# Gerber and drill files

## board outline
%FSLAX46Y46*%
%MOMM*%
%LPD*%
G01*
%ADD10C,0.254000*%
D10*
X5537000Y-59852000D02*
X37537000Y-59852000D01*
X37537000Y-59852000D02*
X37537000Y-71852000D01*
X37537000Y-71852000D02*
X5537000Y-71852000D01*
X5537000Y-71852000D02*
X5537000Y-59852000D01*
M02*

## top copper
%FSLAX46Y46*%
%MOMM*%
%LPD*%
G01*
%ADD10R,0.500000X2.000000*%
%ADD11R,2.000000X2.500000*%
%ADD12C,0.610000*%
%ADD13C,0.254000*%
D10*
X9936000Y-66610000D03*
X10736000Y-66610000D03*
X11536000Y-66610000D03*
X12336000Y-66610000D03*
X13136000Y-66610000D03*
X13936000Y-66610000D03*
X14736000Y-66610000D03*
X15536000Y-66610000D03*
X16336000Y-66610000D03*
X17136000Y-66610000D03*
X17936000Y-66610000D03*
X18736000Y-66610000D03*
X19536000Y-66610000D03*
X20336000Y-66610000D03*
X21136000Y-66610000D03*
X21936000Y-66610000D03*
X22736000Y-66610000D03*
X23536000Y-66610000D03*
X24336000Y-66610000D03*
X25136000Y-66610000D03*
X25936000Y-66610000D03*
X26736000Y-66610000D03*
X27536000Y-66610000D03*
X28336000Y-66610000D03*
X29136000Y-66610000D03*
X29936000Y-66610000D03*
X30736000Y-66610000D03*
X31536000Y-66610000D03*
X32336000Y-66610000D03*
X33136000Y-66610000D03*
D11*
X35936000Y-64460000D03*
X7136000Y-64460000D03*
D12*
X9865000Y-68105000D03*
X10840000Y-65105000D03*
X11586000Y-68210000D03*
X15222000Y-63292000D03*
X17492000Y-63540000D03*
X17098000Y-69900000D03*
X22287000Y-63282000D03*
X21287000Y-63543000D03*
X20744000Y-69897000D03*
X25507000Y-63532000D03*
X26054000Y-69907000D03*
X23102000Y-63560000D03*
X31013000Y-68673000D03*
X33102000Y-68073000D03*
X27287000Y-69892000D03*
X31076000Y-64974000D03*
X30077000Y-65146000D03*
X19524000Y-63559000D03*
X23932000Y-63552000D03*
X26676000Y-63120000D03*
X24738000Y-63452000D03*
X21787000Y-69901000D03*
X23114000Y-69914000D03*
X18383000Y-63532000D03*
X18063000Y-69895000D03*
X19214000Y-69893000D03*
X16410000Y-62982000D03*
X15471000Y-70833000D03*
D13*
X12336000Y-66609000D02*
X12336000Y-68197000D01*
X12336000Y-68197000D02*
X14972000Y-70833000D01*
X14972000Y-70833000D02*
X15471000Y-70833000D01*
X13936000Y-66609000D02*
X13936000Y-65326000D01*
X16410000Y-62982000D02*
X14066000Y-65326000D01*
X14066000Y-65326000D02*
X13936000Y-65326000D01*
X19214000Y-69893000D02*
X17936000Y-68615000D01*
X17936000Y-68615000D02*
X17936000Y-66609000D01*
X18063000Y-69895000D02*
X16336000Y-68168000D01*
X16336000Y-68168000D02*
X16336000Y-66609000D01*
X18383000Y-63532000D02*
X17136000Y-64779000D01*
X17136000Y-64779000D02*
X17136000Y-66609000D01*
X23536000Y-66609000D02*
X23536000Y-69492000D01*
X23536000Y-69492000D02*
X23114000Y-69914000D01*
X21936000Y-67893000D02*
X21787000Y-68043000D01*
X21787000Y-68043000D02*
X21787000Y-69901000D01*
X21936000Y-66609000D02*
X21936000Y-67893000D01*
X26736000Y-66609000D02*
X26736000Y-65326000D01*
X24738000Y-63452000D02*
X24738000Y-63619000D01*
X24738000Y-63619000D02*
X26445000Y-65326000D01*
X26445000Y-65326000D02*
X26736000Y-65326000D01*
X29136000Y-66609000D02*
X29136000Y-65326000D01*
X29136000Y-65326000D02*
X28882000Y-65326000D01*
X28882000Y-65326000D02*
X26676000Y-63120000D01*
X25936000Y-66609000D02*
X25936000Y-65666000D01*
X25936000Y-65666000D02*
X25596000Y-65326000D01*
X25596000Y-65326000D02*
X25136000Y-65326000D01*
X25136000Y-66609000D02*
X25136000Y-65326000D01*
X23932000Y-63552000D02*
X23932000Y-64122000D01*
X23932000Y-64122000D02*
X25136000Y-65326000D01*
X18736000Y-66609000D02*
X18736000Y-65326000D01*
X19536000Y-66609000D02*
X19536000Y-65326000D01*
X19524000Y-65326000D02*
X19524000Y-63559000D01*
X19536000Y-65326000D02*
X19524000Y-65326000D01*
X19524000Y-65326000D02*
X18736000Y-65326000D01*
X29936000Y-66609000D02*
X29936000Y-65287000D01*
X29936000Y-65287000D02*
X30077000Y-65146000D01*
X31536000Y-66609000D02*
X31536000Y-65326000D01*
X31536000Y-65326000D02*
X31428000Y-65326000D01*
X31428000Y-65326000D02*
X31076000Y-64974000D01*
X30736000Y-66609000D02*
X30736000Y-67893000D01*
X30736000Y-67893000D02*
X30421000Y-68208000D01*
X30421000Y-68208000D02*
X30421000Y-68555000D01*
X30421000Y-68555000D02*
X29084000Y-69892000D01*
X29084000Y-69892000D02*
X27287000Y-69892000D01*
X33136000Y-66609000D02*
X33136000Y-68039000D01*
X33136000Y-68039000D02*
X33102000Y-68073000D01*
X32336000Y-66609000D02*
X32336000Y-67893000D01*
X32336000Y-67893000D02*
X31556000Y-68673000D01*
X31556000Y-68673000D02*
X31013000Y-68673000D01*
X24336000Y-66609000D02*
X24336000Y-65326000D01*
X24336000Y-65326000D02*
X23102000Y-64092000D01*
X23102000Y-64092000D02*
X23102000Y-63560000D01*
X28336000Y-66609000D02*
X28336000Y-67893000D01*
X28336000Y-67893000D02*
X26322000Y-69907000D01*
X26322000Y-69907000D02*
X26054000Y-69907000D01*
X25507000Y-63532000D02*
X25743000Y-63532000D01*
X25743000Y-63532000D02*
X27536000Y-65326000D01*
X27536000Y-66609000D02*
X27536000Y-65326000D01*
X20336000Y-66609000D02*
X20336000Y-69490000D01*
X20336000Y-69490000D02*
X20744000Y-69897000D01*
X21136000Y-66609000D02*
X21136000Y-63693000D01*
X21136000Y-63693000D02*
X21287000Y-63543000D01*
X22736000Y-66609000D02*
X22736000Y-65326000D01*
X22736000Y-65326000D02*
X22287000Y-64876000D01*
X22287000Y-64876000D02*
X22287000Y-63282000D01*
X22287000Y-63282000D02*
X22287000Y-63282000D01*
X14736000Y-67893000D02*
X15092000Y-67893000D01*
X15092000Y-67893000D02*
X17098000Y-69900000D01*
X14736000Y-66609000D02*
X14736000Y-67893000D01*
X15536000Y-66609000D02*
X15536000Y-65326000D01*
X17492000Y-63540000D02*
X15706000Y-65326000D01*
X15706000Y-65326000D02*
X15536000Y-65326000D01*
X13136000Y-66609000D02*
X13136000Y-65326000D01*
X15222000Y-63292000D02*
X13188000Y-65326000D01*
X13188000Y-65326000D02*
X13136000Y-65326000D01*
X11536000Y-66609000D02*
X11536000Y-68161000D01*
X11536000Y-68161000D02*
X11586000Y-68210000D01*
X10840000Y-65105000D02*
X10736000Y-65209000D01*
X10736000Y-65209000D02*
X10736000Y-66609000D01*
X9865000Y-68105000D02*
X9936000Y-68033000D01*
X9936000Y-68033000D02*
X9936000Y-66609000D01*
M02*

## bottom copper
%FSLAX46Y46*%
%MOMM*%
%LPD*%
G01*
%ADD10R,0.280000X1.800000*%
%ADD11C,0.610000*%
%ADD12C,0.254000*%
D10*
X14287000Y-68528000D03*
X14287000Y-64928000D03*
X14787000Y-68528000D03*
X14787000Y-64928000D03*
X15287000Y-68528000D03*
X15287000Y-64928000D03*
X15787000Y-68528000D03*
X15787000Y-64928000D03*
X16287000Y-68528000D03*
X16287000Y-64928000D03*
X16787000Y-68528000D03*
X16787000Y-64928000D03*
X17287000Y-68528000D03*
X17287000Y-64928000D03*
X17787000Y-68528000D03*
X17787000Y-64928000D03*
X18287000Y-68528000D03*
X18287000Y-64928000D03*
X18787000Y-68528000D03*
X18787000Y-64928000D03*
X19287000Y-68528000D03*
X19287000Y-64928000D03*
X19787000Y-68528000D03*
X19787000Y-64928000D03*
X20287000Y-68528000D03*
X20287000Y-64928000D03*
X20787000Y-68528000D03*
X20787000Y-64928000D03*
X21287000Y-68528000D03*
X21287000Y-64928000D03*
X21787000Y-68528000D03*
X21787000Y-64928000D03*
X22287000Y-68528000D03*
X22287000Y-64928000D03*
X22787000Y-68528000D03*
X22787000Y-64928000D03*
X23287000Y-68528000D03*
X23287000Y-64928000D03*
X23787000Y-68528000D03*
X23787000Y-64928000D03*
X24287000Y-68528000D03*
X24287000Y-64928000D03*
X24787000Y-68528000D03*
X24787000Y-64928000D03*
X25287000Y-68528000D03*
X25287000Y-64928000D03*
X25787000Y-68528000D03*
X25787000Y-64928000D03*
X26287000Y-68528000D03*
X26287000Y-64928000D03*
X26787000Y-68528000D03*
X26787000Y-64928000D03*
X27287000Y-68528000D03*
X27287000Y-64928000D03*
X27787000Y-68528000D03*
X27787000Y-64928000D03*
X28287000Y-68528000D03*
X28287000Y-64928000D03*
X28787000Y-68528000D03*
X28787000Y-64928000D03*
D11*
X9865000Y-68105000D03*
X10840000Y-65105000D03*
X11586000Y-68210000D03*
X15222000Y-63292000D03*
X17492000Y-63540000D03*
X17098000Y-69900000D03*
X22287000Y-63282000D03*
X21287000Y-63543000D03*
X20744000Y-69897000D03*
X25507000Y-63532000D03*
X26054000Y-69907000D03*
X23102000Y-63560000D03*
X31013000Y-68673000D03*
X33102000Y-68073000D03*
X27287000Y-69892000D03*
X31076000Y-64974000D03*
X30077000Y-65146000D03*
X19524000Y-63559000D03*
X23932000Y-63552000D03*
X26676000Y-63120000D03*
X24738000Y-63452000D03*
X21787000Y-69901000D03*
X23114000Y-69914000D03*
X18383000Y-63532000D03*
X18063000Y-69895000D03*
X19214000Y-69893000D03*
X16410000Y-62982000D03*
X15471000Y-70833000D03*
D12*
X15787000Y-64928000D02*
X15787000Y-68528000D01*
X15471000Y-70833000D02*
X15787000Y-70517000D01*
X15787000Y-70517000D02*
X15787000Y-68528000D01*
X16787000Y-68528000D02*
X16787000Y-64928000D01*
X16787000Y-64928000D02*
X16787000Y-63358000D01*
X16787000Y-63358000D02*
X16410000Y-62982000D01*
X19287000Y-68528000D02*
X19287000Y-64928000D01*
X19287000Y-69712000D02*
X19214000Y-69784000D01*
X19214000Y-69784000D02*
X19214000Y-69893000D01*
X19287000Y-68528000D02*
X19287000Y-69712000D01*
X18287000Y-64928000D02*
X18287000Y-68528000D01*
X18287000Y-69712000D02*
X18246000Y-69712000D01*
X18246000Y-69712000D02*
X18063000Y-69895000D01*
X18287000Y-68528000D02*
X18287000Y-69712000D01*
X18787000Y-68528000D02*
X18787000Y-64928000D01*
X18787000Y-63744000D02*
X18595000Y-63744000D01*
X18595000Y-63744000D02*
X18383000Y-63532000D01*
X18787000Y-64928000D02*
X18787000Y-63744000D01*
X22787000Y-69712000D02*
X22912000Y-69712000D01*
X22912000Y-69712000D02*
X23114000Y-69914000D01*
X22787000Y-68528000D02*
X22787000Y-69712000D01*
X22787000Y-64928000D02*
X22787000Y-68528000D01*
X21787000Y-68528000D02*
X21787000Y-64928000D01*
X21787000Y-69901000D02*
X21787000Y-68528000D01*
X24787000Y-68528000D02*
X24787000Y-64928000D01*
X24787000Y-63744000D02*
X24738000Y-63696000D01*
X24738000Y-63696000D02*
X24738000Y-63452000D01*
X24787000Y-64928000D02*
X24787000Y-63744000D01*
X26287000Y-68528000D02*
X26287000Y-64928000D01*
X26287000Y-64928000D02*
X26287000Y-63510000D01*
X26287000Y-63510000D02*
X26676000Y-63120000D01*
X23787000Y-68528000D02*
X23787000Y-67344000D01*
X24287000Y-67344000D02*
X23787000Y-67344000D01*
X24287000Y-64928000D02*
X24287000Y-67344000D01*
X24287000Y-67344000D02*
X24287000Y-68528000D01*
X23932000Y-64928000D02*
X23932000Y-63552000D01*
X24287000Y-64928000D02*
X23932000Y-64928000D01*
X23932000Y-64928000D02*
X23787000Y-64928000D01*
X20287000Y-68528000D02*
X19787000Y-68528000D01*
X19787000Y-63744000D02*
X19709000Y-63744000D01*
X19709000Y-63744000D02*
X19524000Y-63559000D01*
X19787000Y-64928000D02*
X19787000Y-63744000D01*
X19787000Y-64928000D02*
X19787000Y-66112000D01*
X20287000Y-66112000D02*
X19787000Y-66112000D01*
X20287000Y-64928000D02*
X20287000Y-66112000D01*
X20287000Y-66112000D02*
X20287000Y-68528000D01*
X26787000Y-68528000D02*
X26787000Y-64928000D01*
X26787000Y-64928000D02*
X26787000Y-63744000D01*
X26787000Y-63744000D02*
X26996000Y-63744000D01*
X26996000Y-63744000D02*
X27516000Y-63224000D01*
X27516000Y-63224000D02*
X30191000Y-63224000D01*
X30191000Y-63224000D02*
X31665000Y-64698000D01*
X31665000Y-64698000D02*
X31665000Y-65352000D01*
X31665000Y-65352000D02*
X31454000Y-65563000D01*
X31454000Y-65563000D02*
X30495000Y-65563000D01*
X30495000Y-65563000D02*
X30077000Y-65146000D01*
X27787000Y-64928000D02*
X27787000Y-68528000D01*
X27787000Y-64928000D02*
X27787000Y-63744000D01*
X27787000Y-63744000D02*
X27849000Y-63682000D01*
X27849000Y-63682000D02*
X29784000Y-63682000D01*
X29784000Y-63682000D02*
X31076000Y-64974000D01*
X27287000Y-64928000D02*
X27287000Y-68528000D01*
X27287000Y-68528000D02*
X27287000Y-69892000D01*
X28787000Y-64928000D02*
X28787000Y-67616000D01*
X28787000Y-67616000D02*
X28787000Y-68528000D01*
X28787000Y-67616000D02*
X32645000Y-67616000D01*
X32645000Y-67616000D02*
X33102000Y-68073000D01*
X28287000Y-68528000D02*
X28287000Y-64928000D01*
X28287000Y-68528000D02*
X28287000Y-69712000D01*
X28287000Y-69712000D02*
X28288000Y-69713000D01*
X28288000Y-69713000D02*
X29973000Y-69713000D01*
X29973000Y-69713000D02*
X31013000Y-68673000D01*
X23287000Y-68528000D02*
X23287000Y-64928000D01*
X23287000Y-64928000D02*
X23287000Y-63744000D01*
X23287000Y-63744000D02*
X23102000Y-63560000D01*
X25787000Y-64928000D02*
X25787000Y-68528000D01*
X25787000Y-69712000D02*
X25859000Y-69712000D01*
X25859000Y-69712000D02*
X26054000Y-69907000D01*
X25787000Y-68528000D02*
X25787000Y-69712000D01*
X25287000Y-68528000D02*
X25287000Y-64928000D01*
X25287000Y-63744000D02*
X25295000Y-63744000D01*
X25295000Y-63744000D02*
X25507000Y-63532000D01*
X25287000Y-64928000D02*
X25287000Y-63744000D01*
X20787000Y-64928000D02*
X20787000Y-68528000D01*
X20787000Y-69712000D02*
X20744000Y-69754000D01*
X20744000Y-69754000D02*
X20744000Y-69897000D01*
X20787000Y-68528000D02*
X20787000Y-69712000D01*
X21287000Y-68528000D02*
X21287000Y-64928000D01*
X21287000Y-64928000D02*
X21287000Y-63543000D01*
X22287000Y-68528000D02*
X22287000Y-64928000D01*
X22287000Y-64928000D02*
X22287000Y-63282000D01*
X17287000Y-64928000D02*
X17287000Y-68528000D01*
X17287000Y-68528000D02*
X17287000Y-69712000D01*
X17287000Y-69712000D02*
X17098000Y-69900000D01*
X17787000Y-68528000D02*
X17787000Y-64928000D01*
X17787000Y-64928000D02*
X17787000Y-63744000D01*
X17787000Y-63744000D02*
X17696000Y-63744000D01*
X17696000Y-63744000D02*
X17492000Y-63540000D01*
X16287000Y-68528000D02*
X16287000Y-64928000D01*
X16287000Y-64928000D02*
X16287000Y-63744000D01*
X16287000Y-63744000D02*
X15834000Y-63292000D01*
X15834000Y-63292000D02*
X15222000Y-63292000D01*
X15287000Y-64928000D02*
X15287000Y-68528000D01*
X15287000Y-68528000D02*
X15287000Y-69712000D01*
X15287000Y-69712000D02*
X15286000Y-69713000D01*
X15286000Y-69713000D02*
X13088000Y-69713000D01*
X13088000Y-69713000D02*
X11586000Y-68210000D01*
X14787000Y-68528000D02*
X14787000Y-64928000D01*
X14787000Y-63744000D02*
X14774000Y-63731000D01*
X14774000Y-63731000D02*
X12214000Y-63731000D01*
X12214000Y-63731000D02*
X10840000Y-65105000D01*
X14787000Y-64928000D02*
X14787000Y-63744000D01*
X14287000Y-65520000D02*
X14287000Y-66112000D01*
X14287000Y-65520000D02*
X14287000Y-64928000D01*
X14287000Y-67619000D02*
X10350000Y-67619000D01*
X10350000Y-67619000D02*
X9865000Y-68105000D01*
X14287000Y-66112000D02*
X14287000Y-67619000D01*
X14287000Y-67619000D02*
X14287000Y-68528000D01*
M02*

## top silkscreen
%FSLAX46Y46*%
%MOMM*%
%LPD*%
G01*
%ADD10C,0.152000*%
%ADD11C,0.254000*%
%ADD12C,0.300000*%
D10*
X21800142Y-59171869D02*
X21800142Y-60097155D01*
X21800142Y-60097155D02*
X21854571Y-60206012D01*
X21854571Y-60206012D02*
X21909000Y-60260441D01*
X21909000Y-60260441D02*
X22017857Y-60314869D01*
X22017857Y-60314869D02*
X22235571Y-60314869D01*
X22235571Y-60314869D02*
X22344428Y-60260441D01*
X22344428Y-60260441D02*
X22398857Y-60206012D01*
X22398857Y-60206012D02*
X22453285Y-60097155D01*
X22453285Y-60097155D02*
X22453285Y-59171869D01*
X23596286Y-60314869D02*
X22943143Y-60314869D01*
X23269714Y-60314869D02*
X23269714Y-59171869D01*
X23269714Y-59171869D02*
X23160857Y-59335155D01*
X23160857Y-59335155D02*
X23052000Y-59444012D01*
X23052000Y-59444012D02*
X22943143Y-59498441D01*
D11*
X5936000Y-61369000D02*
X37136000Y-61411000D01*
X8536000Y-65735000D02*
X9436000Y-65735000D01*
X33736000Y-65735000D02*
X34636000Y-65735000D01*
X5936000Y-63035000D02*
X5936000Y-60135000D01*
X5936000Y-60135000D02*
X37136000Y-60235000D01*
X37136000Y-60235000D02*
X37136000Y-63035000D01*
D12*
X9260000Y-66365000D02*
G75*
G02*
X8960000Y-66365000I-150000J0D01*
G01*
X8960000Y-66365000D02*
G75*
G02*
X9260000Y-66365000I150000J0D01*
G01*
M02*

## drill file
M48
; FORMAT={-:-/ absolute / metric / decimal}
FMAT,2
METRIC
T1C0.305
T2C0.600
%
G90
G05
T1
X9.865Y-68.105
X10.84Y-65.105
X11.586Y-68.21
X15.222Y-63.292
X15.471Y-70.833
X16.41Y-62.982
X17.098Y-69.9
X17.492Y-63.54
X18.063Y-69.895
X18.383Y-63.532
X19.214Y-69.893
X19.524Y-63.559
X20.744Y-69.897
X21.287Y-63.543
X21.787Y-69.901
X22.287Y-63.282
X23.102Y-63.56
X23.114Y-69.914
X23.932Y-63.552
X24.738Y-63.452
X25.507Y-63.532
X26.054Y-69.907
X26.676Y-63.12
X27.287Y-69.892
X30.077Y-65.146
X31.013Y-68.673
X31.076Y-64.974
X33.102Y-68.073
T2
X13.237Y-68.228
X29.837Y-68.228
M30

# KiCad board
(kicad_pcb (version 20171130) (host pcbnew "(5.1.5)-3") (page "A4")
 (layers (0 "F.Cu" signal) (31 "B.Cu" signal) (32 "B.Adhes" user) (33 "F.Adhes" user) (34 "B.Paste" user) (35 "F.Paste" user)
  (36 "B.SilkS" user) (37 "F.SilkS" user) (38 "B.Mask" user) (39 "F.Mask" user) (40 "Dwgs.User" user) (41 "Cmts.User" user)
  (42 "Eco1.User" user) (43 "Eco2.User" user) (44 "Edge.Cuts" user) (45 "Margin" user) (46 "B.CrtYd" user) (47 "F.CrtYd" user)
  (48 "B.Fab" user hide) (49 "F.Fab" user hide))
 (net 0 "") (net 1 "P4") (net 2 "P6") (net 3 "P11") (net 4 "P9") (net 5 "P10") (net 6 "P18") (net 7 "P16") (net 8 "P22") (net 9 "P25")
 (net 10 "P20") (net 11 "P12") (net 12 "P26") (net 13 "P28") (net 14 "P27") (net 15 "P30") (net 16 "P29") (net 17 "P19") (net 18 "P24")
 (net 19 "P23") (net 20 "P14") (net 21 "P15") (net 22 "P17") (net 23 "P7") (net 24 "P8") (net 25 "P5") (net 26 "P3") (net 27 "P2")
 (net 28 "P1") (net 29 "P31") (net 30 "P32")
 (segment (start 15.787 64.928) (end 15.787 68.528) (width 0.254) (layer "B.Cu") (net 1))
 (segment (start 15.471 70.833) (end 15.787 70.517) (width 0.254) (layer "B.Cu") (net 1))
 (segment (start 15.787 70.517) (end 15.787 68.528) (width 0.254) (layer "B.Cu") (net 1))
 (segment (start 16.787 68.528) (end 16.787 64.928) (width 0.254) (layer "B.Cu") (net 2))
 (segment (start 16.787 64.928) (end 16.787 63.358) (width 0.254) (layer "B.Cu") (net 2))
 (segment (start 16.787 63.358) (end 16.41 62.982) (width 0.254) (layer "B.Cu") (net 2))
 (segment (start 19.287 68.528) (end 19.287 64.928) (width 0.254) (layer "B.Cu") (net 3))
 (segment (start 19.287 69.712) (end 19.214 69.784) (width 0.254) (layer "B.Cu") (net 3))
 (segment (start 19.214 69.784) (end 19.214 69.893) (width 0.254) (layer "B.Cu") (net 3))
 (segment (start 19.287 68.528) (end 19.287 69.712) (width 0.254) (layer "B.Cu") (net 3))
 (segment (start 18.287 64.928) (end 18.287 68.528) (width 0.254) (layer "B.Cu") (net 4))
 (segment (start 18.287 69.712) (end 18.246 69.712) (width 0.254) (layer "B.Cu") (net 4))
 (segment (start 18.246 69.712) (end 18.063 69.895) (width 0.254) (layer "B.Cu") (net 4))
 (segment (start 18.287 68.528) (end 18.287 69.712) (width 0.254) (layer "B.Cu") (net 4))
 (segment (start 18.787 68.528) (end 18.787 64.928) (width 0.254) (layer "B.Cu") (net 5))
 (segment (start 18.787 63.744) (end 18.595 63.744) (width 0.254) (layer "B.Cu") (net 5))
 (segment (start 18.595 63.744) (end 18.383 63.532) (width 0.254) (layer "B.Cu") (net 5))
 (segment (start 18.787 64.928) (end 18.787 63.744) (width 0.254) (layer "B.Cu") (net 5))
 (segment (start 22.787 69.712) (end 22.912 69.712) (width 0.254) (layer "B.Cu") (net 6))
 (segment (start 22.912 69.712) (end 23.114 69.914) (width 0.254) (layer "B.Cu") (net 6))
 (segment (start 22.787 68.528) (end 22.787 69.712) (width 0.254) (layer "B.Cu") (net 6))
 (segment (start 22.787 64.928) (end 22.787 68.528) (width 0.254) (layer "B.Cu") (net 6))
 (segment (start 21.787 68.528) (end 21.787 64.928) (width 0.254) (layer "B.Cu") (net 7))
 (segment (start 21.787 69.901) (end 21.787 68.528) (width 0.254) (layer "B.Cu") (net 7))
 (segment (start 24.787 68.528) (end 24.787 64.928) (width 0.254) (layer "B.Cu") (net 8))
 (segment (start 24.787 63.744) (end 24.738 63.696) (width 0.254) (layer "B.Cu") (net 8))
 (segment (start 24.738 63.696) (end 24.738 63.452) (width 0.254) (layer "B.Cu") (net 8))
 (segment (start 24.787 64.928) (end 24.787 63.744) (width 0.254) (layer "B.Cu") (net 8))
 (segment (start 26.287 68.528) (end 26.287 64.928) (width 0.254) (layer "B.Cu") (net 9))
 (segment (start 26.287 64.928) (end 26.287 63.51) (width 0.254) (layer "B.Cu") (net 9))
 (segment (start 26.287 63.51) (end 26.676 63.12) (width 0.254) (layer "B.Cu") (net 9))
 (segment (start 23.787 68.528) (end 23.787 67.344) (width 0.254) (layer "B.Cu") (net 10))
 (segment (start 24.287 67.344) (end 23.787 67.344) (width 0.254) (layer "B.Cu") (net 10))
 (segment (start 24.287 64.928) (end 24.287 67.344) (width 0.254) (layer "B.Cu") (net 10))
 (segment (start 24.287 67.344) (end 24.287 68.528) (width 0.254) (layer "B.Cu") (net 10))
 (segment (start 23.932 64.928) (end 23.932 63.552) (width 0.254) (layer "B.Cu") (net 10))
 (segment (start 24.287 64.928) (end 23.932 64.928) (width 0.254) (layer "B.Cu") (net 10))
 (segment (start 23.932 64.928) (end 23.787 64.928) (width 0.254) (layer "B.Cu") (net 10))
 (segment (start 20.287 68.528) (end 19.787 68.528) (width 0.254) (layer "B.Cu") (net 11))
 (segment (start 19.787 63.744) (end 19.709 63.744) (width 0.254) (layer "B.Cu") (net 11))
 (segment (start 19.709 63.744) (end 19.524 63.559) (width 0.254) (layer "B.Cu") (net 11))
 (segment (start 19.787 64.928) (end 19.787 63.744) (width 0.254) (layer "B.Cu") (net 11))
 (segment (start 19.787 64.928) (end 19.787 66.112) (width 0.254) (layer "B.Cu") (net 11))
 (segment (start 20.287 66.112) (end 19.787 66.112) (width 0.254) (layer "B.Cu") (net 11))
 (segment (start 20.287 64.928) (end 20.287 66.112) (width 0.254) (layer "B.Cu") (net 11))
 (segment (start 20.287 66.112) (end 20.287 68.528) (width 0.254) (layer "B.Cu") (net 11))
 (segment (start 26.787 68.528) (end 26.787 64.928) (width 0.254) (layer "B.Cu") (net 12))
 (segment (start 26.787 64.928) (end 26.787 63.744) (width 0.254) (layer "B.Cu") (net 12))
 (segment (start 26.787 63.744) (end 26.996 63.744) (width 0.254) (layer "B.Cu") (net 12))
 (segment (start 26.996 63.744) (end 27.516 63.224) (width 0.254) (layer "B.Cu") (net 12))
 (segment (start 27.516 63.224) (end 30.191 63.224) (width 0.254) (layer "B.Cu") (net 12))
 (segment (start 30.191 63.224) (end 31.665 64.698) (width 0.254) (layer "B.Cu") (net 12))
 (segment (start 31.665 64.698) (end 31.665 65.352) (width 0.254) (layer "B.Cu") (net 12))
 (segment (start 31.665 65.352) (end 31.454 65.563) (width 0.254) (layer "B.Cu") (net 12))
 (segment (start 31.454 65.563) (end 30.495 65.563) (width 0.254) (layer "B.Cu") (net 12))
 (segment (start 30.495 65.563) (end 30.077 65.146) (width 0.254) (layer "B.Cu") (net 12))
 (segment (start 27.787 64.928) (end 27.787 68.528) (width 0.254) (layer "B.Cu") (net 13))
 (segment (start 27.787 64.928) (end 27.787 63.744) (width 0.254) (layer "B.Cu") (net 13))
 (segment (start 27.787 63.744) (end 27.849 63.682) (width 0.254) (layer "B.Cu") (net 13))
 (segment (start 27.849 63.682) (end 29.784 63.682) (width 0.254) (layer "B.Cu") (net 13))
 (segment (start 29.784 63.682) (end 31.076 64.974) (width 0.254) (layer "B.Cu") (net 13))
 (segment (start 27.287 64.928) (end 27.287 68.528) (width 0.254) (layer "B.Cu") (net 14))
 (segment (start 27.287 68.528) (end 27.287 69.892) (width 0.254) (layer "B.Cu") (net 14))
 (segment (start 28.787 64.928) (end 28.787 67.616) (width 0.254) (layer "B.Cu") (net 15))
 (segment (start 28.787 67.616) (end 28.787 68.528) (width 0.254) (layer "B.Cu") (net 15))
 (segment (start 28.787 67.616) (end 32.645 67.616) (width 0.254) (layer "B.Cu") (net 15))
 (segment (start 32.645 67.616) (end 33.102 68.073) (width 0.254) (layer "B.Cu") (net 15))
 (segment (start 28.287 68.528) (end 28.287 64.928) (width 0.254) (layer "B.Cu") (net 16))
 (segment (start 28.287 68.528) (end 28.287 69.712) (width 0.254) (layer "B.Cu") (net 16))
 (segment (start 28.287 69.712) (end 28.288 69.713) (width 0.254) (layer "B.Cu") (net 16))
 (segment (start 28.288 69.713) (end 29.973 69.713) (width 0.254) (layer "B.Cu") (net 16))
 (segment (start 29.973 69.713) (end 31.013 68.673) (width 0.254) (layer "B.Cu") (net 16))
 (segment (start 23.287 68.528) (end 23.287 64.928) (width 0.254) (layer "B.Cu") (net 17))
 (segment (start 23.287 64.928) (end 23.287 63.744) (width 0.254) (layer "B.Cu") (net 17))
 (segment (start 23.287 63.744) (end 23.102 63.56) (width 0.254) (layer "B.Cu") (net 17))
 (segment (start 25.787 64.928) (end 25.787 68.528) (width 0.254) (layer "B.Cu") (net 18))
 (segment (start 25.787 69.712) (end 25.859 69.712) (width 0.254) (layer "B.Cu") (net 18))
 (segment (start 25.859 69.712) (end 26.054 69.907) (width 0.254) (layer "B.Cu") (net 18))
 (segment (start 25.787 68.528) (end 25.787 69.712) (width 0.254) (layer "B.Cu") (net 18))
 (segment (start 25.287 68.528) (end 25.287 64.928) (width 0.254) (layer "B.Cu") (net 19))
 (segment (start 25.287 63.744) (end 25.295 63.744) (width 0.254) (layer "B.Cu") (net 19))
 (segment (start 25.295 63.744) (end 25.507 63.532) (width 0.254) (layer "B.Cu") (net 19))
 (segment (start 25.287 64.928) (end 25.287 63.744) (width 0.254) (layer "B.Cu") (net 19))
 (segment (start 20.787 64.928) (end 20.787 68.528) (width 0.254) (layer "B.Cu") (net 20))
 (segment (start 20.787 69.712) (end 20.744 69.754) (width 0.254) (layer "B.Cu") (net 20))
 (segment (start 20.744 69.754) (end 20.744 69.897) (width 0.254) (layer "B.Cu") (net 20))
 (segment (start 20.787 68.528) (end 20.787 69.712) (width 0.254) (layer "B.Cu") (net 20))
 (segment (start 21.287 68.528) (end 21.287 64.928) (width 0.254) (layer "B.Cu") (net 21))
 (segment (start 21.287 64.928) (end 21.287 63.543) (width 0.254) (layer "B.Cu") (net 21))
 (segment (start 22.287 68.528) (end 22.287 64.928) (width 0.254) (layer "B.Cu") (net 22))
 (segment (start 22.287 64.928) (end 22.287 63.282) (width 0.254) (layer "B.Cu") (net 22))
 (segment (start 17.287 64.928) (end 17.287 68.528) (width 0.254) (layer "B.Cu") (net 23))
 (segment (start 17.287 68.528) (end 17.287 69.712) (width 0.254) (layer "B.Cu") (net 23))
 (segment (start 17.287 69.712) (end 17.098 69.9) (width 0.254) (layer "B.Cu") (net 23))
 (segment (start 17.787 68.528) (end 17.787 64.928) (width 0.254) (layer "B.Cu") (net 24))
 (segment (start 17.787 64.928) (end 17.787 63.744) (width 0.254) (layer "B.Cu") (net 24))
 (segment (start 17.787 63.744) (end 17.696 63.744) (width 0.254) (layer "B.Cu") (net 24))
 (segment (start 17.696 63.744) (end 17.492 63.54) (width 0.254) (layer "B.Cu") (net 24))
 (segment (start 16.287 68.528) (end 16.287 64.928) (width 0.254) (layer "B.Cu") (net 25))
 (segment (start 16.287 64.928) (end 16.287 63.744) (width 0.254) (layer "B.Cu") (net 25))
 (segment (start 16.287 63.744) (end 15.834 63.292) (width 0.254) (layer "B.Cu") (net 25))
 (segment (start 15.834 63.292) (end 15.222 63.292) (width 0.254) (layer "B.Cu") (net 25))
 (segment (start 15.287 64.928) (end 15.287 68.528) (width 0.254) (layer "B.Cu") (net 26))
 (segment (start 15.287 68.528) (end 15.287 69.712) (width 0.254) (layer "B.Cu") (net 26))
 (segment (start 15.287 69.712) (end 15.286 69.713) (width 0.254) (layer "B.Cu") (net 26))
 (segment (start 15.286 69.713) (end 13.088 69.713) (width 0.254) (layer "B.Cu") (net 26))
 (segment (start 13.088 69.713) (end 11.586 68.21) (width 0.254) (layer "B.Cu") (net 26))
 (segment (start 14.787 68.528) (end 14.787 64.928) (width 0.254) (layer "B.Cu") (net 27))
 (segment (start 14.787 63.744) (end 14.774 63.731) (width 0.254) (layer "B.Cu") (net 27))
 (segment (start 14.774 63.731) (end 12.214 63.731) (width 0.254) (layer "B.Cu") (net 27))
 (segment (start 12.214 63.731) (end 10.84 65.105) (width 0.254) (layer "B.Cu") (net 27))
 (segment (start 14.787 64.928) (end 14.787 63.744) (width 0.254) (layer "B.Cu") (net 27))
 (segment (start 14.287 65.52) (end 14.287 66.112) (width 0.254) (layer "B.Cu") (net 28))
 (segment (start 14.287 65.52) (end 14.287 64.928) (width 0.254) (layer "B.Cu") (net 28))
 (segment (start 14.287 67.619) (end 10.35 67.619) (width 0.254) (layer "B.Cu") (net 28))
 (segment (start 10.35 67.619) (end 9.865 68.105) (width 0.254) (layer "B.Cu") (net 28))
 (segment (start 14.287 66.112) (end 14.287 67.619) (width 0.254) (layer "B.Cu") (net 28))
 (segment (start 14.287 67.619) (end 14.287 68.528) (width 0.254) (layer "B.Cu") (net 28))
 (gr_line (start 5.537 59.852) (end 37.537 59.852) (width 0.254) (layer "Edge.Cuts"))
 (gr_line (start 37.537 59.852) (end 37.537 71.852) (width 0.254) (layer "Edge.Cuts"))
 (gr_line (start 37.537 71.852) (end 5.537 71.852) (width 0.254) (layer "Edge.Cuts"))
 (gr_line (start 5.537 71.852) (end 5.537 59.852) (width 0.254) (layer "Edge.Cuts"))
 (segment (start 12.336 66.609) (end 12.336 68.197) (width 0.254) (layer "F.Cu") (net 1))
 (segment (start 12.336 68.197) (end 14.972 70.833) (width 0.254) (layer "F.Cu") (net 1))
 (segment (start 14.972 70.833) (end 15.471 70.833) (width 0.254) (layer "F.Cu") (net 1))
 (segment (start 13.936 66.609) (end 13.936 65.326) (width 0.254) (layer "F.Cu") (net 2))
 (segment (start 16.41 62.982) (end 14.066 65.326) (width 0.254) (layer "F.Cu") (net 2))
 (segment (start 14.066 65.326) (end 13.936 65.326) (width 0.254) (layer "F.Cu") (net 2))
 (segment (start 19.214 69.893) (end 17.936 68.615) (width 0.254) (layer "F.Cu") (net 3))
 (segment (start 17.936 68.615) (end 17.936 66.609) (width 0.254) (layer "F.Cu") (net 3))
 (segment (start 18.063 69.895) (end 16.336 68.168) (width 0.254) (layer "F.Cu") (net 4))
 (segment (start 16.336 68.168) (end 16.336 66.609) (width 0.254) (layer "F.Cu") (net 4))
 (segment (start 18.383 63.532) (end 17.136 64.779) (width 0.254) (layer "F.Cu") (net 5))
 (segment (start 17.136 64.779) (end 17.136 66.609) (width 0.254) (layer "F.Cu") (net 5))
 (segment (start 23.536 66.609) (end 23.536 69.492) (width 0.254) (layer "F.Cu") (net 6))
 (segment (start 23.536 69.492) (end 23.114 69.914) (width 0.254) (layer "F.Cu") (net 6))
 (segment (start 21.936 67.893) (end 21.787 68.043) (width 0.254) (layer "F.Cu") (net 7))
 (segment (start 21.787 68.043) (end 21.787 69.901) (width 0.254) (layer "F.Cu") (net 7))
 (segment (start 21.936 66.609) (end 21.936 67.893) (width 0.254) (layer "F.Cu") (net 7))
 (segment (start 26.736 66.609) (end 26.736 65.326) (width 0.254) (layer "F.Cu") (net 8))
 (segment (start 24.738 63.452) (end 24.738 63.619) (width 0.254) (layer "F.Cu") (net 8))
 (segment (start 24.738 63.619) (end 26.445 65.326) (width 0.254) (layer "F.Cu") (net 8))
 (segment (start 26.445 65.326) (end 26.736 65.326) (width 0.254) (layer "F.Cu") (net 8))
 (segment (start 29.136 66.609) (end 29.136 65.326) (width 0.254) (layer "F.Cu") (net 9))
 (segment (start 29.136 65.326) (end 28.882 65.326) (width 0.254) (layer "F.Cu") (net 9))
 (segment (start 28.882 65.326) (end 26.676 63.12) (width 0.254) (layer "F.Cu") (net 9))
 (segment (start 25.936 66.609) (end 25.936 65.666) (width 0.254) (layer "F.Cu") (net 10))
 (segment (start 25.936 65.666) (end 25.596 65.326) (width 0.254) (layer "F.Cu") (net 10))
 (segment (start 25.596 65.326) (end 25.136 65.326) (width 0.254) (layer "F.Cu") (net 10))
 (segment (start 25.136 66.609) (end 25.136 65.326) (width 0.254) (layer "F.Cu") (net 10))
 (segment (start 23.932 63.552) (end 23.932 64.122) (width 0.254) (layer "F.Cu") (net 10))
 (segment (start 23.932 64.122) (end 25.136 65.326) (width 0.254) (layer "F.Cu") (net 10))
 (segment (start 18.736 66.609) (end 18.736 65.326) (width 0.254) (layer "F.Cu") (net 11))
 (segment (start 19.536 66.609) (end 19.536 65.326) (width 0.254) (layer "F.Cu") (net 11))
 (segment (start 19.524 65.326) (end 19.524 63.559) (width 0.254) (layer "F.Cu") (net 11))
 (segment (start 19.536 65.326) (end 19.524 65.326) (width 0.254) (layer "F.Cu") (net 11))
 (segment (start 19.524 65.326) (end 18.736 65.326) (width 0.254) (layer "F.Cu") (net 11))
 (segment (start 29.936 66.609) (end 29.936 65.287) (width 0.254) (layer "F.Cu") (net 12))
 (segment (start 29.936 65.287) (end 30.077 65.146) (width 0.254) (layer "F.Cu") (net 12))
 (segment (start 31.536 66.609) (end 31.536 65.326) (width 0.254) (layer "F.Cu") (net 13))
 (segment (start 31.536 65.326) (end 31.428 65.326) (width 0.254) (layer "F.Cu") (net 13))
 (segment (start 31.428 65.326) (end 31.076 64.974) (width 0.254) (layer "F.Cu") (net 13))
 (segment (start 30.736 66.609) (end 30.736 67.893) (width 0.254) (layer "F.Cu") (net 14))
 (segment (start 30.736 67.893) (end 30.421 68.208) (width 0.254) (layer "F.Cu") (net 14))
 (segment (start 30.421 68.208) (end 30.421 68.555) (width 0.254) (layer "F.Cu") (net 14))
 (segment (start 30.421 68.555) (end 29.084 69.892) (width 0.254) (layer "F.Cu") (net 14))
 (segment (start 29.084 69.892) (end 27.287 69.892) (width 0.254) (layer "F.Cu") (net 14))
 (segment (start 33.136 66.609) (end 33.136 68.039) (width 0.254) (layer "F.Cu") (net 15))
 (segment (start 33.136 68.039) (end 33.102 68.073) (width 0.254) (layer "F.Cu") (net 15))
 (segment (start 32.336 66.609) (end 32.336 67.893) (width 0.254) (layer "F.Cu") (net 16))
 (segment (start 32.336 67.893) (end 31.556 68.673) (width 0.254) (layer "F.Cu") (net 16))
 (segment (start 31.556 68.673) (end 31.013 68.673) (width 0.254) (layer "F.Cu") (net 16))
 (segment (start 24.336 66.609) (end 24.336 65.326) (width 0.254) (layer "F.Cu") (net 17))
 (segment (start 24.336 65.326) (end 23.102 64.092) (width 0.254) (layer "F.Cu") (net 17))
 (segment (start 23.102 64.092) (end 23.102 63.56) (width 0.254) (layer "F.Cu") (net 17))
 (segment (start 28.336 66.609) (end 28.336 67.893) (width 0.254) (layer "F.Cu") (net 18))
 (segment (start 28.336 67.893) (end 26.322 69.907) (width 0.254) (layer "F.Cu") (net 18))
 (segment (start 26.322 69.907) (end 26.054 69.907) (width 0.254) (layer "F.Cu") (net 18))
 (segment (start 25.507 63.532) (end 25.743 63.532) (width 0.254) (layer "F.Cu") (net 19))
 (segment (start 25.743 63.532) (end 27.536 65.326) (width 0.254) (layer "F.Cu") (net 19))
 (segment (start 27.536 66.609) (end 27.536 65.326) (width 0.254) (layer "F.Cu") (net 19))
 (segment (start 20.336 66.609) (end 20.336 69.49) (width 0.254) (layer "F.Cu") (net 20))
 (segment (start 20.336 69.49) (end 20.744 69.897) (width 0.254) (layer "F.Cu") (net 20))
 (segment (start 21.136 66.609) (end 21.136 63.693) (width 0.254) (layer "F.Cu") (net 21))
 (segment (start 21.136 63.693) (end 21.287 63.543) (width 0.254) (layer "F.Cu") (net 21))
 (segment (start 22.736 66.609) (end 22.736 65.326) (width 0.254) (layer "F.Cu") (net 22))
 (segment (start 22.736 65.326) (end 22.287 64.876) (width 0.254) (layer "F.Cu") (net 22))
 (segment (start 22.287 64.876) (end 22.287 63.282) (width 0.254) (layer "F.Cu") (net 22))
 (segment (start 22.287 63.282) (end 22.287 63.282) (width 0.254) (layer "F.Cu") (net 22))
 (segment (start 14.736 67.893) (end 15.092 67.893) (width 0.254) (layer "F.Cu") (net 23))
 (segment (start 15.092 67.893) (end 17.098 69.9) (width 0.254) (layer "F.Cu") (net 23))
 (segment (start 14.736 66.609) (end 14.736 67.893) (width 0.254) (layer "F.Cu") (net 23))
 (segment (start 15.536 66.609) (end 15.536 65.326) (width 0.254) (layer "F.Cu") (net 24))
 (segment (start 17.492 63.54) (end 15.706 65.326) (width 0.254) (layer "F.Cu") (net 24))
 (segment (start 15.706 65.326) (end 15.536 65.326) (width 0.254) (layer "F.Cu") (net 24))
 (segment (start 13.136 66.609) (end 13.136 65.326) (width 0.254) (layer "F.Cu") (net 25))
 (segment (start 15.222 63.292) (end 13.188 65.326) (width 0.254) (layer "F.Cu") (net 25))
 (segment (start 13.188 65.326) (end 13.136 65.326) (width 0.254) (layer "F.Cu") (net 25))
 (segment (start 11.536 66.609) (end 11.536 68.161) (width 0.254) (layer "F.Cu") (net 26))
 (segment (start 11.536 68.161) (end 11.586 68.21) (width 0.254) (layer "F.Cu") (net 26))
 (segment (start 10.84 65.105) (end 10.736 65.209) (width 0.254) (layer "F.Cu") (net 27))
 (segment (start 10.736 65.209) (end 10.736 66.609) (width 0.254) (layer "F.Cu") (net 27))
 (segment (start 9.865 68.105) (end 9.936 68.033) (width 0.254) (layer "F.Cu") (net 28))
 (segment (start 9.936 68.033) (end 9.936 66.609) (width 0.254) (layer "F.Cu") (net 28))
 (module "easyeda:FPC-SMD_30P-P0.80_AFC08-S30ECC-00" (layer "F.Cu") (at 21.536 65.535)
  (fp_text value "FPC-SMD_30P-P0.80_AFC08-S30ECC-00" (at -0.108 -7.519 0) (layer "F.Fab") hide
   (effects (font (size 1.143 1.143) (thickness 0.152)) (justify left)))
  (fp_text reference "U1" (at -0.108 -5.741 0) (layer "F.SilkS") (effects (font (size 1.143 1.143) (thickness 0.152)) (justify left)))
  (fp_line (start -15.6 -4.166) (end 15.6 -4.124) (width 0.254) (layer "F.SilkS"))
  (fp_line (start -13 0.2) (end -12.1 0.2) (width 0.254) (layer "F.SilkS"))
  (fp_line (start 12.2 0.2) (end 13.1 0.2) (width 0.254) (layer "F.SilkS"))
  (fp_line (start -15.6 -2.5) (end -15.6 -5.4) (width 0.254) (layer "F.SilkS"))
  (fp_line (start -15.6 -5.4) (end 15.6 -5.3) (width 0.254) (layer "F.SilkS"))
  (fp_line (start 15.6 -5.3) (end 15.6 -2.5) (width 0.254) (layer "F.SilkS"))
  (fp_circle (center -12.426 0.83) (end -12.276 0.83) (layer "F.SilkS") (width 0.3))
  (pad 1 smd rect (at -11.6 1.075 180) (size 0.5 2) (layers "F.Cu" "F.Paste" "F.Mask") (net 28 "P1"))
  (pad 2 smd rect (at -10.8 1.075 180) (size 0.5 2) (layers "F.Cu" "F.Paste" "F.Mask") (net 27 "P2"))
  (pad 3 smd rect (at -10 1.075 180) (size 0.5 2) (layers "F.Cu" "F.Paste" "F.Mask") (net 26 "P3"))
  (pad 4 smd rect (at -9.2 1.075 180) (size 0.5 2) (layers "F.Cu" "F.Paste" "F.Mask") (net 1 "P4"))
  (pad 5 smd rect (at -8.4 1.075 180) (size 0.5 2) (layers "F.Cu" "F.Paste" "F.Mask") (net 25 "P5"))
  (pad 6 smd rect (at -7.6 1.075 180) (size 0.5 2) (layers "F.Cu" "F.Paste" "F.Mask") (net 2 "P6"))
  (pad 7 smd rect (at -6.8 1.075 180) (size 0.5 2) (layers "F.Cu" "F.Paste" "F.Mask") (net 23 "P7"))
  (pad 8 smd rect (at -6 1.075 180) (size 0.5 2) (layers "F.Cu" "F.Paste" "F.Mask") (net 24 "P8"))
  (pad 9 smd rect (at -5.2 1.075 180) (size 0.5 2) (layers "F.Cu" "F.Paste" "F.Mask") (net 4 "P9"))
  (pad 10 smd rect (at -4.4 1.075 180) (size 0.5 2) (layers "F.Cu" "F.Paste" "F.Mask") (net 5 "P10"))
  (pad 11 smd rect (at -3.6 1.075 180) (size 0.5 2) (layers "F.Cu" "F.Paste" "F.Mask") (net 3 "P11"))
  (pad 12 smd rect (at -2.8 1.075 180) (size 0.5 2) (layers "F.Cu" "F.Paste" "F.Mask") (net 11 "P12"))
  (pad 13 smd rect (at -2 1.075 180) (size 0.5 2) (layers "F.Cu" "F.Paste" "F.Mask") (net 11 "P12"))
  (pad 14 smd rect (at -1.2 1.075 180) (size 0.5 2) (layers "F.Cu" "F.Paste" "F.Mask") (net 20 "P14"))
  (pad 15 smd rect (at -0.4 1.075 180) (size 0.5 2) (layers "F.Cu" "F.Paste" "F.Mask") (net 21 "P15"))
  (pad 16 smd rect (at 0.4 1.075 180) (size 0.5 2) (layers "F.Cu" "F.Paste" "F.Mask") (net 7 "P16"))
  (pad 17 smd rect (at 1.2 1.075 180) (size 0.5 2) (layers "F.Cu" "F.Paste" "F.Mask") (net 22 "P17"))
  (pad 18 smd rect (at 2 1.075 180) (size 0.5 2) (layers "F.Cu" "F.Paste" "F.Mask") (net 6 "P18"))
  (pad 19 smd rect (at 2.8 1.075 180) (size 0.5 2) (layers "F.Cu" "F.Paste" "F.Mask") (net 17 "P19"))
  (pad 20 smd rect (at 3.6 1.075 180) (size 0.5 2) (layers "F.Cu" "F.Paste" "F.Mask") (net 10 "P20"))
  (pad 21 smd rect (at 4.4 1.075 180) (size 0.5 2) (layers "F.Cu" "F.Paste" "F.Mask") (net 10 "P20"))
  (pad 22 smd rect (at 5.2 1.075 180) (size 0.5 2) (layers "F.Cu" "F.Paste" "F.Mask") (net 8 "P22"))
  (pad 23 smd rect (at 6 1.075 180) (size 0.5 2) (layers "F.Cu" "F.Paste" "F.Mask") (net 19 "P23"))
  (pad 24 smd rect (at 6.8 1.075 180) (size 0.5 2) (layers "F.Cu" "F.Paste" "F.Mask") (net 18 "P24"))
  (pad 25 smd rect (at 7.6 1.075 180) (size 0.5 2) (layers "F.Cu" "F.Paste" "F.Mask") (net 9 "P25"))
  (pad 26 smd rect (at 8.4 1.075 180) (size 0.5 2) (layers "F.Cu" "F.Paste" "F.Mask") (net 12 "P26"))
  (pad 27 smd rect (at 9.2 1.075 180) (size 0.5 2) (layers "F.Cu" "F.Paste" "F.Mask") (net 14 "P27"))
  (pad 28 smd rect (at 10 1.075 180) (size 0.5 2) (layers "F.Cu" "F.Paste" "F.Mask") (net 13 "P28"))
  (pad 29 smd rect (at 10.8 1.075 180) (size 0.5 2) (layers "F.Cu" "F.Paste" "F.Mask") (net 16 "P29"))
  (pad 30 smd rect (at 11.6 1.075 180) (size 0.5 2) (layers "F.Cu" "F.Paste" "F.Mask") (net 15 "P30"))
  (pad 31 smd rect (at 14.4 -1.075 180) (size 2 2.5) (layers "F.Cu" "F.Paste" "F.Mask") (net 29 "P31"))
  (pad 32 smd rect (at -14.4 -1.075 180) (size 2 2.5) (layers "F.Cu" "F.Paste" "F.Mask") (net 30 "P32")))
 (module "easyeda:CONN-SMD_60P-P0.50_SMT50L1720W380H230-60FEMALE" (layer "F.Cu") (at 21.537 66.728)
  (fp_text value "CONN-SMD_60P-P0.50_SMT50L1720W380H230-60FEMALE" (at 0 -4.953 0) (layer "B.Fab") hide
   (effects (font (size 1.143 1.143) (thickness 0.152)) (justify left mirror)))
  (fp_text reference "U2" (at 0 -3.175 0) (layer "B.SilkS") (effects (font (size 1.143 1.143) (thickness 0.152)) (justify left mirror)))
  (pad 1 smd rect (at -7.25 1.8 180) (size 0.28 1.8) (layers "B.Cu" "B.Paste" "B.Mask") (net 28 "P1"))
  (pad 2 smd rect (at -7.25 -1.8 180) (size 0.28 1.8) (layers "B.Cu" "B.Paste" "B.Mask") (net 28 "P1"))
  (pad 3 smd rect (at -6.75 1.8 180) (size 0.28 1.8) (layers "B.Cu" "B.Paste" "B.Mask") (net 27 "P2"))
  (pad 4 smd rect (at -6.75 -1.8 180) (size 0.28 1.8) (layers "B.Cu" "B.Paste" "B.Mask") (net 27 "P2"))
  (pad 5 smd rect (at -6.25 1.8 180) (size 0.28 1.8) (layers "B.Cu" "B.Paste" "B.Mask") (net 26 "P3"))
  (pad 6 smd rect (at -6.25 -1.8 180) (size 0.28 1.8) (layers "B.Cu" "B.Paste" "B.Mask") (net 26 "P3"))
  (pad 7 smd rect (at -5.75 1.8 180) (size 0.28 1.8) (layers "B.Cu" "B.Paste" "B.Mask") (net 1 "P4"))
  (pad 8 smd rect (at -5.75 -1.8 180) (size 0.28 1.8) (layers "B.Cu" "B.Paste" "B.Mask") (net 1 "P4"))
  (pad 9 smd rect (at -5.25 1.8 180) (size 0.28 1.8) (layers "B.Cu" "B.Paste" "B.Mask") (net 25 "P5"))
  (pad 10 smd rect (at -5.25 -1.8 180) (size 0.28 1.8) (layers "B.Cu" "B.Paste" "B.Mask") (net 25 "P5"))
  (pad 11 smd rect (at -4.75 1.8 180) (size 0.28 1.8) (layers "B.Cu" "B.Paste" "B.Mask") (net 2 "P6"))
  (pad 12 smd rect (at -4.75 -1.8 180) (size 0.28 1.8) (layers "B.Cu" "B.Paste" "B.Mask") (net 2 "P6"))
  (pad 13 smd rect (at -4.25 1.8 180) (size 0.28 1.8) (layers "B.Cu" "B.Paste" "B.Mask") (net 23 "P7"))
  (pad 14 smd rect (at -4.25 -1.8 180) (size 0.28 1.8) (layers "B.Cu" "B.Paste" "B.Mask") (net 23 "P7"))
  (pad 15 smd rect (at -3.75 1.8 180) (size 0.28 1.8) (layers "B.Cu" "B.Paste" "B.Mask") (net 24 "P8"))
  (pad 16 smd rect (at -3.75 -1.8 180) (size 0.28 1.8) (layers "B.Cu" "B.Paste" "B.Mask") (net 24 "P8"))
  (pad 17 smd rect (at -3.25 1.8 180) (size 0.28 1.8) (layers "B.Cu" "B.Paste" "B.Mask") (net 4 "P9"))
  (pad 18 smd rect (at -3.25 -1.8 180) (size 0.28 1.8) (layers "B.Cu" "B.Paste" "B.Mask") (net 4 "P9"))
  (pad 19 smd rect (at -2.75 1.8 180) (size 0.28 1.8) (layers "B.Cu" "B.Paste" "B.Mask") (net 5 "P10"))
  (pad 20 smd rect (at -2.75 -1.8 180) (size 0.28 1.8) (layers "B.Cu" "B.Paste" "B.Mask") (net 5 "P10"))
  (pad 21 smd rect (at -2.25 1.8 180) (size 0.28 1.8) (layers "B.Cu" "B.Paste" "B.Mask") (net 3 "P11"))
  (pad 22 smd rect (at -2.25 -1.8 180) (size 0.28 1.8) (layers "B.Cu" "B.Paste" "B.Mask") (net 3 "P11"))
  (pad 23 smd rect (at -1.75 1.8 180) (size 0.28 1.8) (layers "B.Cu" "B.Paste" "B.Mask") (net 11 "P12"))
  (pad 24 smd rect (at -1.75 -1.8 180) (size 0.28 1.8) (layers "B.Cu" "B.Paste" "B.Mask") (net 11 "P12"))
  (pad 25 smd rect (at -1.25 1.8 180) (size 0.28 1.8) (layers "B.Cu" "B.Paste" "B.Mask") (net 11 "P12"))
  (pad 26 smd rect (at -1.25 -1.8 180) (size 0.28 1.8) (layers "B.Cu" "B.Paste" "B.Mask") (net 11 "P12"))
  (pad 27 smd rect (at -0.75 1.8 180) (size 0.28 1.8) (layers "B.Cu" "B.Paste" "B.Mask") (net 20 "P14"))
  (pad 28 smd rect (at -0.75 -1.8 180) (size 0.28 1.8) (layers "B.Cu" "B.Paste" "B.Mask") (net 20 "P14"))
  (pad 29 smd rect (at -0.25 1.8 180) (size 0.28 1.8) (layers "B.Cu" "B.Paste" "B.Mask") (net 21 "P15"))
  (pad 30 smd rect (at -0.25 -1.8 180) (size 0.28 1.8) (layers "B.Cu" "B.Paste" "B.Mask") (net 21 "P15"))
  (pad 31 smd rect (at 0.25 1.8 180) (size 0.28 1.8) (layers "B.Cu" "B.Paste" "B.Mask") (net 7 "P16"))
  (pad 32 smd rect (at 0.25 -1.8 180) (size 0.28 1.8) (layers "B.Cu" "B.Paste" "B.Mask") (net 7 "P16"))
  (pad 33 smd rect (at 0.75 1.8 180) (size 0.28 1.8) (layers "B.Cu" "B.Paste" "B.Mask") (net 22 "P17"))
  (pad 34 smd rect (at 0.75 -1.8 180) (size 0.28 1.8) (layers "B.Cu" "B.Paste" "B.Mask") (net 22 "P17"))
  (pad 35 smd rect (at 1.25 1.8 180) (size 0.28 1.8) (layers "B.Cu" "B.Paste" "B.Mask") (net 6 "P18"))
  (pad 36 smd rect (at 1.25 -1.8 180) (size 0.28 1.8) (layers "B.Cu" "B.Paste" "B.Mask") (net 6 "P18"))
  (pad 37 smd rect (at 1.75 1.8 180) (size 0.28 1.8) (layers "B.Cu" "B.Paste" "B.Mask") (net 17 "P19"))
  (pad 38 smd rect (at 1.75 -1.8 180) (size 0.28 1.8) (layers "B.Cu" "B.Paste" "B.Mask") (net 17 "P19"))
  (pad 39 smd rect (at 2.25 1.8 180) (size 0.28 1.8) (layers "B.Cu" "B.Paste" "B.Mask") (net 10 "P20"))
  (pad 40 smd rect (at 2.25 -1.8 180) (size 0.28 1.8) (layers "B.Cu" "B.Paste" "B.Mask") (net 10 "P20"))
  (pad 41 smd rect (at 2.75 1.8 180) (size 0.28 1.8) (layers "B.Cu" "B.Paste" "B.Mask") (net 10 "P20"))
  (pad 42 smd rect (at 2.75 -1.8 180) (size 0.28 1.8) (layers "B.Cu" "B.Paste" "B.Mask") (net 10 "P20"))
  (pad 43 smd rect (at 3.25 1.8 180) (size 0.28 1.8) (layers "B.Cu" "B.Paste" "B.Mask") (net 8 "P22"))
  (pad 44 smd rect (at 3.25 -1.8 180) (size 0.28 1.8) (layers "B.Cu" "B.Paste" "B.Mask") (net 8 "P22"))
  (pad 45 smd rect (at 3.75 1.8 180) (size 0.28 1.8) (layers "B.Cu" "B.Paste" "B.Mask") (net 19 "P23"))
  (pad 46 smd rect (at 3.75 -1.8 180) (size 0.28 1.8) (layers "B.Cu" "B.Paste" "B.Mask") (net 19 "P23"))
  (pad 47 smd rect (at 4.25 1.8 180) (size 0.28 1.8) (layers "B.Cu" "B.Paste" "B.Mask") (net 18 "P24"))
  (pad 48 smd rect (at 4.25 -1.8 180) (size 0.28 1.8) (layers "B.Cu" "B.Paste" "B.Mask") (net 18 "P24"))
  (pad 49 smd rect (at 4.75 1.8 180) (size 0.28 1.8) (layers "B.Cu" "B.Paste" "B.Mask") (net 9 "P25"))
  (pad 50 smd rect (at 4.75 -1.8 180) (size 0.28 1.8) (layers "B.Cu" "B.Paste" "B.Mask") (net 9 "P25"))
  (pad 51 smd rect (at 5.25 1.8 180) (size 0.28 1.8) (layers "B.Cu" "B.Paste" "B.Mask") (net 12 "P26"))
  (pad 52 smd rect (at 5.25 -1.8 180) (size 0.28 1.8) (layers "B.Cu" "B.Paste" "B.Mask") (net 12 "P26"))
  (pad 53 smd rect (at 5.75 1.8 180) (size 0.28 1.8) (layers "B.Cu" "B.Paste" "B.Mask") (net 14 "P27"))
  (pad 54 smd rect (at 5.75 -1.8 180) (size 0.28 1.8) (layers "B.Cu" "B.Paste" "B.Mask") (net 14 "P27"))
  (pad 55 smd rect (at 6.25 1.8 180) (size 0.28 1.8) (layers "B.Cu" "B.Paste" "B.Mask") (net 13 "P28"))
  (pad 56 smd rect (at 6.25 -1.8 180) (size 0.28 1.8) (layers "B.Cu" "B.Paste" "B.Mask") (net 13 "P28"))
  (pad 57 smd rect (at 6.75 1.8 180) (size 0.28 1.8) (layers "B.Cu" "B.Paste" "B.Mask") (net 16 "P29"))
  (pad 58 smd rect (at 6.75 -1.8 180) (size 0.28 1.8) (layers "B.Cu" "B.Paste" "B.Mask") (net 16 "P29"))
  (pad 59 smd rect (at 7.25 1.8 180) (size 0.28 1.8) (layers "B.Cu" "B.Paste" "B.Mask") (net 15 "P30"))
  (pad 60 smd rect (at 7.25 -1.8 180) (size 0.28 1.8) (layers "B.Cu" "B.Paste" "B.Mask") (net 15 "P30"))
  (pad "" np_thru_hole circle (at 8.3 1.5) (size 0.6 0.6) (drill 0.6) (layers "*.Cu" "*.Mask"))
  (pad "" np_thru_hole circle (at -8.3 1.5) (size 0.6 0.6) (drill 0.6) (layers "*.Cu" "*.Mask")))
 (via (at 9.865 68.105) (size 0.61) (drill 0.305) (layers "F.Cu" "B.Cu") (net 28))
 (via (at 10.84 65.105) (size 0.61) (drill 0.305) (layers "F.Cu" "B.Cu") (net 27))
 (via (at 11.586 68.21) (size 0.61) (drill 0.305) (layers "F.Cu" "B.Cu") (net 26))
 (via (at 15.222 63.292) (size 0.61) (drill 0.305) (layers "F.Cu" "B.Cu") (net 25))
 (via (at 17.492 63.54) (size 0.61) (drill 0.305) (layers "F.Cu" "B.Cu") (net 24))
 (via (at 17.098 69.9) (size 0.61) (drill 0.305) (layers "F.Cu" "B.Cu") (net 23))
 (via (at 22.287 63.282) (size 0.61) (drill 0.305) (layers "F.Cu" "B.Cu") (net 22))
 (via (at 21.287 63.543) (size 0.61) (drill 0.305) (layers "F.Cu" "B.Cu") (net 21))
 (via (at 20.744 69.897) (size 0.61) (drill 0.305) (layers "F.Cu" "B.Cu") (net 20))
 (via (at 25.507 63.532) (size 0.61) (drill 0.305) (layers "F.Cu" "B.Cu") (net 19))
 (via (at 26.054 69.907) (size 0.61) (drill 0.305) (layers "F.Cu" "B.Cu") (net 18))
 (via (at 23.102 63.56) (size 0.61) (drill 0.305) (layers "F.Cu" "B.Cu") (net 17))
 (via (at 31.013 68.673) (size 0.61) (drill 0.305) (layers "F.Cu" "B.Cu") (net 16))
 (via (at 33.102 68.073) (size 0.61) (drill 0.305) (layers "F.Cu" "B.Cu") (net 15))
 (via (at 27.287 69.892) (size 0.61) (drill 0.305) (layers "F.Cu" "B.Cu") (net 14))
 (via (at 31.076 64.974) (size 0.61) (drill 0.305) (layers "F.Cu" "B.Cu") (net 13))
 (via (at 30.077 65.146) (size 0.61) (drill 0.305) (layers "F.Cu" "B.Cu") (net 12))
 (via (at 19.524 63.559) (size 0.61) (drill 0.305) (layers "F.Cu" "B.Cu") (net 11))
 (via (at 23.932 63.552) (size 0.61) (drill 0.305) (layers "F.Cu" "B.Cu") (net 10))
 (via (at 26.676 63.12) (size 0.61) (drill 0.305) (layers "F.Cu" "B.Cu") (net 9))
 (via (at 24.738 63.452) (size 0.61) (drill 0.305) (layers "F.Cu" "B.Cu") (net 8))
 (via (at 21.787 69.901) (size 0.61) (drill 0.305) (layers "F.Cu" "B.Cu") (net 7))
 (via (at 23.114 69.914) (size 0.61) (drill 0.305) (layers "F.Cu" "B.Cu") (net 6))
 (via (at 18.383 63.532) (size 0.61) (drill 0.305) (layers "F.Cu" "B.Cu") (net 5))
 (via (at 18.063 69.895) (size 0.61) (drill 0.305) (layers "F.Cu" "B.Cu") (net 4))
 (via (at 19.214 69.893) (size 0.61) (drill 0.305) (layers "F.Cu" "B.Cu") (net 3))
 (via (at 16.41 62.982) (size 0.61) (drill 0.305) (layers "F.Cu" "B.Cu") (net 2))
 (via (at 15.471 70.833) (size 0.61) (drill 0.305) (layers "F.Cu" "B.Cu") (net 1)))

